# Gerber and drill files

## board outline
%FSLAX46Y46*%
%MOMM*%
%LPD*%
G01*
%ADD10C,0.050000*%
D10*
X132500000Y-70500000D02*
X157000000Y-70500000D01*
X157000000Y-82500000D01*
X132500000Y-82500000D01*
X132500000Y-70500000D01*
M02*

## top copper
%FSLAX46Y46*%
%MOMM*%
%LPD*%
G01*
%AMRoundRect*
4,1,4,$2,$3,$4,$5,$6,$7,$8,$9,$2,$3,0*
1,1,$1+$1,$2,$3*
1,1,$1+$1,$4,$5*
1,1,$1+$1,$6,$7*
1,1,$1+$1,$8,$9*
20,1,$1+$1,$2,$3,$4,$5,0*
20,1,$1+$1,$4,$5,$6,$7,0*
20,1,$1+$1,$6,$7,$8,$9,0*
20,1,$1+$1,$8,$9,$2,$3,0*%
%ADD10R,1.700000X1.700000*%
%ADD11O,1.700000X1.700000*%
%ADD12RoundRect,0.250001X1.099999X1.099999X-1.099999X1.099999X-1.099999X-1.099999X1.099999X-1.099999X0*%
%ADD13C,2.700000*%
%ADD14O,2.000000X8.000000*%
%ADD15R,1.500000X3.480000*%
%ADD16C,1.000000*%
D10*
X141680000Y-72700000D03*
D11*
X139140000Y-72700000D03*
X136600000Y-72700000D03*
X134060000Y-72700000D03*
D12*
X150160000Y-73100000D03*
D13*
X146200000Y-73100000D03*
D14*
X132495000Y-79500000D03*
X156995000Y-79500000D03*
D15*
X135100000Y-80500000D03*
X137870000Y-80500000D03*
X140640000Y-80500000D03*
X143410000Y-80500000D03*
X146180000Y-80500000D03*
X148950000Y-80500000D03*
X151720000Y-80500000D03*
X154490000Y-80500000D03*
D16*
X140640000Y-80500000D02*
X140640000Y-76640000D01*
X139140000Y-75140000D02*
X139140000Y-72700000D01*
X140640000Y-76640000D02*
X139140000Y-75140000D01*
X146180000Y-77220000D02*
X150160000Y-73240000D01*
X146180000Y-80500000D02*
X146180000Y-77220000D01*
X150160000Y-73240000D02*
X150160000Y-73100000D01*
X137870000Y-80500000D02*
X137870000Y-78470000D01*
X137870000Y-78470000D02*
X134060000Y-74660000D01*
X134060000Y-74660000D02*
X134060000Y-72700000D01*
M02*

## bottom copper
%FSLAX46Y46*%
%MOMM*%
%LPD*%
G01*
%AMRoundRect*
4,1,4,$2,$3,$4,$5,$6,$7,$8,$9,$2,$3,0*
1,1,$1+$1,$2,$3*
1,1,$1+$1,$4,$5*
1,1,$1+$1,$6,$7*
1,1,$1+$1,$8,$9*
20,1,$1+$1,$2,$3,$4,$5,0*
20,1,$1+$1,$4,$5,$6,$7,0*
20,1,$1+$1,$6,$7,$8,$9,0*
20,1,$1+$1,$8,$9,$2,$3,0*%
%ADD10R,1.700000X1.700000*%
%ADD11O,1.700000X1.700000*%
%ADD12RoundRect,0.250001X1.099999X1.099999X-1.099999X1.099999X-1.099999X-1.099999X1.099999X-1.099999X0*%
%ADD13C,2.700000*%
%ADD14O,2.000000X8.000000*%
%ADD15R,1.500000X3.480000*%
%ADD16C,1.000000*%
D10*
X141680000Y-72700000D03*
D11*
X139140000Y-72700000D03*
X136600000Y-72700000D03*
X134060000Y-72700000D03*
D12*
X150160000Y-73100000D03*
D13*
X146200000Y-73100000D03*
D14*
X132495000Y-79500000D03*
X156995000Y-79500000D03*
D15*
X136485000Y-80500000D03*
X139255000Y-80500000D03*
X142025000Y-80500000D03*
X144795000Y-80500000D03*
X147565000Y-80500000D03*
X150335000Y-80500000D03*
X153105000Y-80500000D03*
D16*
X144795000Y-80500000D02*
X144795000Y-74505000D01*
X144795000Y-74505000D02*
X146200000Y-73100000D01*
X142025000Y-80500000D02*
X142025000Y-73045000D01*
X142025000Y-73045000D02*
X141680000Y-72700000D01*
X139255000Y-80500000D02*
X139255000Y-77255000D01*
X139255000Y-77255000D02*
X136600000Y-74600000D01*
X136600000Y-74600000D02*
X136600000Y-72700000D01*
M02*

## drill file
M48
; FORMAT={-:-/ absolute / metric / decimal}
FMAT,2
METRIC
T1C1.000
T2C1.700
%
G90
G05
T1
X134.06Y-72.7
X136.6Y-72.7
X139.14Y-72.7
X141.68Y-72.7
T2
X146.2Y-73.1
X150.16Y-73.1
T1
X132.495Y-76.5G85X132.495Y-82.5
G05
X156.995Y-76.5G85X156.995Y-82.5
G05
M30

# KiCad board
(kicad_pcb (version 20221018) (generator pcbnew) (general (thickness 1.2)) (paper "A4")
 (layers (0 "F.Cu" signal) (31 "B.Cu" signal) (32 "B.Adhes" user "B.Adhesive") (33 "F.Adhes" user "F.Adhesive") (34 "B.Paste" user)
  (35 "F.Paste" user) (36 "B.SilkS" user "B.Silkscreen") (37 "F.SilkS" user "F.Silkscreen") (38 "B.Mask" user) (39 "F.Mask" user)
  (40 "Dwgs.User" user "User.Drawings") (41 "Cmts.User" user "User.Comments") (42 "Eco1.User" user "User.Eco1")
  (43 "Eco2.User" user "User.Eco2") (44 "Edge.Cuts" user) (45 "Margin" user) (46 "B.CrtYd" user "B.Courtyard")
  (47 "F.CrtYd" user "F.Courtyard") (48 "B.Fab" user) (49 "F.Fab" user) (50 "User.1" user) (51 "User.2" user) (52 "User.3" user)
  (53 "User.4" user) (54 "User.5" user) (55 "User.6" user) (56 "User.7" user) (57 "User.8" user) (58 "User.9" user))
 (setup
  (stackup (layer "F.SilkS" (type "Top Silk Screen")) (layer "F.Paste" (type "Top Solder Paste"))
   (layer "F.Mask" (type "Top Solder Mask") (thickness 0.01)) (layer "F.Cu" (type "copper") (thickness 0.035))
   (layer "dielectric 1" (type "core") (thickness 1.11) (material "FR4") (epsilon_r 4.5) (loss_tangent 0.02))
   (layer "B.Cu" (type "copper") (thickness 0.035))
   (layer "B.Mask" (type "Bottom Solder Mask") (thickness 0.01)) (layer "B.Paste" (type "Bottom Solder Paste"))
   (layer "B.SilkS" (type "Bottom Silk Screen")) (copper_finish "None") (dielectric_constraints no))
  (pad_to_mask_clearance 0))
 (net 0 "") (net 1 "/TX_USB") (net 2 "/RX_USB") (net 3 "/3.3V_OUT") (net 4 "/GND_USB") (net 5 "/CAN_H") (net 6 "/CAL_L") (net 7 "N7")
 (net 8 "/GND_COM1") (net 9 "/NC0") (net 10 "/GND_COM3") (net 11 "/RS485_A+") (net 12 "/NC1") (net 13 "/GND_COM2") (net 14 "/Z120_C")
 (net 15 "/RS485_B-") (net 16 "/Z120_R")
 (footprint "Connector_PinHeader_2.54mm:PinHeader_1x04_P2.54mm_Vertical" (layer "F.Cu") (at 141.68 72.7 -90)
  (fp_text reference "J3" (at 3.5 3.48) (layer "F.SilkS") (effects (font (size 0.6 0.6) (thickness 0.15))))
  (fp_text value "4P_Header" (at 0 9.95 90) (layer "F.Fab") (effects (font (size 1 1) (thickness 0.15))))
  (pad "1" thru_hole rect (at 0 0 270) (size 1.7 1.7) (drill 1) (layers "*.Cu" "*.Mask") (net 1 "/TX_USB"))
  (pad "2" thru_hole oval (at 0 2.54 270) (size 1.7 1.7) (drill 1) (layers "*.Cu" "*.Mask") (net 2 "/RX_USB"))
  (pad "3" thru_hole oval (at 0 5.08 270) (size 1.7 1.7) (drill 1) (layers "*.Cu" "*.Mask") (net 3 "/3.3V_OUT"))
  (pad "4" thru_hole oval (at 0 7.62 270) (size 1.7 1.7) (drill 1) (layers "*.Cu" "*.Mask") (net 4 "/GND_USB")))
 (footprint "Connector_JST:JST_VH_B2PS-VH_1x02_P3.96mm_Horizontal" (layer "F.Cu") (at 150.16 73.1 180)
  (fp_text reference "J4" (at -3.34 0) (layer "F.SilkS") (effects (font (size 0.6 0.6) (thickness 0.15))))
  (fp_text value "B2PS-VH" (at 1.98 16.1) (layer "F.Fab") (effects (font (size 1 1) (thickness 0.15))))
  (pad "1" thru_hole roundrect (at 0 0 180) (size 2.7 2.7) (drill 1.7) (layers "*.Cu" "*.Mask") (roundrect_rratio 0.092593) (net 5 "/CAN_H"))
  (pad "2" thru_hole circle (at 3.96 0 180) (size 2.7 2.7) (drill 1.7) (layers "*.Cu" "*.Mask") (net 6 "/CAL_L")))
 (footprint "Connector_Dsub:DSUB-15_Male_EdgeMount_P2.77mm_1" (layer "F.Cu") (at 144.795 80.5)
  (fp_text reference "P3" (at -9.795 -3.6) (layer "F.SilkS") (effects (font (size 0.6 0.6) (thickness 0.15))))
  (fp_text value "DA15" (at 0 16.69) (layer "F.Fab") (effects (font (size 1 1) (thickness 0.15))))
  (pad "0" thru_hole oval (at -12.3 -1) (size 2 8) (drill oval 1 7) (layers "*.Cu" "*.Mask") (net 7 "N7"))
  (pad "0" thru_hole oval (at 12.2 -1) (size 2 8) (drill oval 1 7) (layers "*.Cu" "*.Mask") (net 7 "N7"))
  (pad "1" smd rect (at -9.695 0) (size 1.5 3.48) (layers "F.Cu" "F.Paste" "F.Mask") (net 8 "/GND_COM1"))
  (pad "2" smd rect (at -6.925 0) (size 1.5 3.48) (layers "F.Cu" "F.Paste" "F.Mask") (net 4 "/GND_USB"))
  (pad "3" smd rect (at -4.155 0) (size 1.5 3.48) (layers "F.Cu" "F.Paste" "F.Mask") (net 2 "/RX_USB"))
  (pad "4" smd rect (at -1.385 0) (size 1.5 3.48) (layers "F.Cu" "F.Paste" "F.Mask") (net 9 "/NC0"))
  (pad "5" smd rect (at 1.385 0) (size 1.5 3.48) (layers "F.Cu" "F.Paste" "F.Mask") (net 5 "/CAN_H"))
  (pad "6" smd rect (at 4.155 0) (size 1.5 3.48) (layers "F.Cu" "F.Paste" "F.Mask") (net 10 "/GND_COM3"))
  (pad "7" smd rect (at 6.925 0) (size 1.5 3.48) (layers "F.Cu" "F.Paste" "F.Mask") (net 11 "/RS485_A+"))
  (pad "8" smd rect (at 9.695 0) (size 1.5 3.48) (layers "F.Cu" "F.Paste" "F.Mask") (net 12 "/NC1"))
  (pad "9" smd rect (at -8.31 0) (size 1.5 3.48) (layers "B.Cu" "B.Paste" "B.Mask") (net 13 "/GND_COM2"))
  (pad "10" smd rect (at -5.54 0) (size 1.5 3.48) (layers "B.Cu" "B.Paste" "B.Mask") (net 3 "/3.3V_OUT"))
  (pad "11" smd rect (at -2.77 0) (size 1.5 3.48) (layers "B.Cu" "B.Paste" "B.Mask") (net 1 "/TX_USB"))
  (pad "12" smd rect (at 0 0) (size 1.5 3.48) (layers "B.Cu" "B.Paste" "B.Mask") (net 6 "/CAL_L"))
  (pad "13" smd rect (at 2.77 0) (size 1.5 3.48) (layers "B.Cu" "B.Paste" "B.Mask") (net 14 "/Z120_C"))
  (pad "14" smd rect (at 5.54 0) (size 1.5 3.48) (layers "B.Cu" "B.Paste" "B.Mask") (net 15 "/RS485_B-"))
  (pad "15" smd rect (at 8.31 0) (size 1.5 3.48) (layers "B.Cu" "B.Paste" "B.Mask") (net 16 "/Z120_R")))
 (gr_rect (start 132.5 70.5) (end 157 82.5) (stroke (width 0.05) (type default)) (fill none) (layer "Edge.Cuts"))
 (segment (start 140.64 80.5) (end 140.64 76.64) (width 1) (layer "F.Cu") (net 2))
 (segment (start 139.14 75.14) (end 139.14 72.7) (width 1) (layer "F.Cu") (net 2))
 (segment (start 140.64 76.64) (end 139.14 75.14) (width 1) (layer "F.Cu") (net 2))
 (segment (start 146.18 77.22) (end 150.16 73.24) (width 1) (layer "F.Cu") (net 5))
 (segment (start 146.18 80.5) (end 146.18 77.22) (width 1) (layer "F.Cu") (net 5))
 (segment (start 150.16 73.24) (end 150.16 73.1) (width 1) (layer "F.Cu") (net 5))
 (segment (start 144.795 80.5) (end 144.795 74.505) (width 1) (layer "B.Cu") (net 6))
 (segment (start 144.795 74.505) (end 146.2 73.1) (width 1) (layer "B.Cu") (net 6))
 (segment (start 142.025 80.5) (end 142.025 73.045) (width 1) (layer "B.Cu") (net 1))
 (segment (start 142.025 73.045) (end 141.68 72.7) (width 1) (layer "B.Cu") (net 1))
 (segment (start 139.255 80.5) (end 139.255 77.255) (width 1) (layer "B.Cu") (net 3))
 (segment (start 139.255 77.255) (end 136.6 74.6) (width 1) (layer "B.Cu") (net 3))
 (segment (start 136.6 74.6) (end 136.6 72.7) (width 1) (layer "B.Cu") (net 3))
 (segment (start 137.87 80.5) (end 137.87 78.47) (width 1) (layer "F.Cu") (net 4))
 (segment (start 137.87 78.47) (end 134.06 74.66) (width 1) (layer "F.Cu") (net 4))
 (segment (start 134.06 74.66) (end 134.06 72.7) (width 1) (layer "F.Cu") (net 4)))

